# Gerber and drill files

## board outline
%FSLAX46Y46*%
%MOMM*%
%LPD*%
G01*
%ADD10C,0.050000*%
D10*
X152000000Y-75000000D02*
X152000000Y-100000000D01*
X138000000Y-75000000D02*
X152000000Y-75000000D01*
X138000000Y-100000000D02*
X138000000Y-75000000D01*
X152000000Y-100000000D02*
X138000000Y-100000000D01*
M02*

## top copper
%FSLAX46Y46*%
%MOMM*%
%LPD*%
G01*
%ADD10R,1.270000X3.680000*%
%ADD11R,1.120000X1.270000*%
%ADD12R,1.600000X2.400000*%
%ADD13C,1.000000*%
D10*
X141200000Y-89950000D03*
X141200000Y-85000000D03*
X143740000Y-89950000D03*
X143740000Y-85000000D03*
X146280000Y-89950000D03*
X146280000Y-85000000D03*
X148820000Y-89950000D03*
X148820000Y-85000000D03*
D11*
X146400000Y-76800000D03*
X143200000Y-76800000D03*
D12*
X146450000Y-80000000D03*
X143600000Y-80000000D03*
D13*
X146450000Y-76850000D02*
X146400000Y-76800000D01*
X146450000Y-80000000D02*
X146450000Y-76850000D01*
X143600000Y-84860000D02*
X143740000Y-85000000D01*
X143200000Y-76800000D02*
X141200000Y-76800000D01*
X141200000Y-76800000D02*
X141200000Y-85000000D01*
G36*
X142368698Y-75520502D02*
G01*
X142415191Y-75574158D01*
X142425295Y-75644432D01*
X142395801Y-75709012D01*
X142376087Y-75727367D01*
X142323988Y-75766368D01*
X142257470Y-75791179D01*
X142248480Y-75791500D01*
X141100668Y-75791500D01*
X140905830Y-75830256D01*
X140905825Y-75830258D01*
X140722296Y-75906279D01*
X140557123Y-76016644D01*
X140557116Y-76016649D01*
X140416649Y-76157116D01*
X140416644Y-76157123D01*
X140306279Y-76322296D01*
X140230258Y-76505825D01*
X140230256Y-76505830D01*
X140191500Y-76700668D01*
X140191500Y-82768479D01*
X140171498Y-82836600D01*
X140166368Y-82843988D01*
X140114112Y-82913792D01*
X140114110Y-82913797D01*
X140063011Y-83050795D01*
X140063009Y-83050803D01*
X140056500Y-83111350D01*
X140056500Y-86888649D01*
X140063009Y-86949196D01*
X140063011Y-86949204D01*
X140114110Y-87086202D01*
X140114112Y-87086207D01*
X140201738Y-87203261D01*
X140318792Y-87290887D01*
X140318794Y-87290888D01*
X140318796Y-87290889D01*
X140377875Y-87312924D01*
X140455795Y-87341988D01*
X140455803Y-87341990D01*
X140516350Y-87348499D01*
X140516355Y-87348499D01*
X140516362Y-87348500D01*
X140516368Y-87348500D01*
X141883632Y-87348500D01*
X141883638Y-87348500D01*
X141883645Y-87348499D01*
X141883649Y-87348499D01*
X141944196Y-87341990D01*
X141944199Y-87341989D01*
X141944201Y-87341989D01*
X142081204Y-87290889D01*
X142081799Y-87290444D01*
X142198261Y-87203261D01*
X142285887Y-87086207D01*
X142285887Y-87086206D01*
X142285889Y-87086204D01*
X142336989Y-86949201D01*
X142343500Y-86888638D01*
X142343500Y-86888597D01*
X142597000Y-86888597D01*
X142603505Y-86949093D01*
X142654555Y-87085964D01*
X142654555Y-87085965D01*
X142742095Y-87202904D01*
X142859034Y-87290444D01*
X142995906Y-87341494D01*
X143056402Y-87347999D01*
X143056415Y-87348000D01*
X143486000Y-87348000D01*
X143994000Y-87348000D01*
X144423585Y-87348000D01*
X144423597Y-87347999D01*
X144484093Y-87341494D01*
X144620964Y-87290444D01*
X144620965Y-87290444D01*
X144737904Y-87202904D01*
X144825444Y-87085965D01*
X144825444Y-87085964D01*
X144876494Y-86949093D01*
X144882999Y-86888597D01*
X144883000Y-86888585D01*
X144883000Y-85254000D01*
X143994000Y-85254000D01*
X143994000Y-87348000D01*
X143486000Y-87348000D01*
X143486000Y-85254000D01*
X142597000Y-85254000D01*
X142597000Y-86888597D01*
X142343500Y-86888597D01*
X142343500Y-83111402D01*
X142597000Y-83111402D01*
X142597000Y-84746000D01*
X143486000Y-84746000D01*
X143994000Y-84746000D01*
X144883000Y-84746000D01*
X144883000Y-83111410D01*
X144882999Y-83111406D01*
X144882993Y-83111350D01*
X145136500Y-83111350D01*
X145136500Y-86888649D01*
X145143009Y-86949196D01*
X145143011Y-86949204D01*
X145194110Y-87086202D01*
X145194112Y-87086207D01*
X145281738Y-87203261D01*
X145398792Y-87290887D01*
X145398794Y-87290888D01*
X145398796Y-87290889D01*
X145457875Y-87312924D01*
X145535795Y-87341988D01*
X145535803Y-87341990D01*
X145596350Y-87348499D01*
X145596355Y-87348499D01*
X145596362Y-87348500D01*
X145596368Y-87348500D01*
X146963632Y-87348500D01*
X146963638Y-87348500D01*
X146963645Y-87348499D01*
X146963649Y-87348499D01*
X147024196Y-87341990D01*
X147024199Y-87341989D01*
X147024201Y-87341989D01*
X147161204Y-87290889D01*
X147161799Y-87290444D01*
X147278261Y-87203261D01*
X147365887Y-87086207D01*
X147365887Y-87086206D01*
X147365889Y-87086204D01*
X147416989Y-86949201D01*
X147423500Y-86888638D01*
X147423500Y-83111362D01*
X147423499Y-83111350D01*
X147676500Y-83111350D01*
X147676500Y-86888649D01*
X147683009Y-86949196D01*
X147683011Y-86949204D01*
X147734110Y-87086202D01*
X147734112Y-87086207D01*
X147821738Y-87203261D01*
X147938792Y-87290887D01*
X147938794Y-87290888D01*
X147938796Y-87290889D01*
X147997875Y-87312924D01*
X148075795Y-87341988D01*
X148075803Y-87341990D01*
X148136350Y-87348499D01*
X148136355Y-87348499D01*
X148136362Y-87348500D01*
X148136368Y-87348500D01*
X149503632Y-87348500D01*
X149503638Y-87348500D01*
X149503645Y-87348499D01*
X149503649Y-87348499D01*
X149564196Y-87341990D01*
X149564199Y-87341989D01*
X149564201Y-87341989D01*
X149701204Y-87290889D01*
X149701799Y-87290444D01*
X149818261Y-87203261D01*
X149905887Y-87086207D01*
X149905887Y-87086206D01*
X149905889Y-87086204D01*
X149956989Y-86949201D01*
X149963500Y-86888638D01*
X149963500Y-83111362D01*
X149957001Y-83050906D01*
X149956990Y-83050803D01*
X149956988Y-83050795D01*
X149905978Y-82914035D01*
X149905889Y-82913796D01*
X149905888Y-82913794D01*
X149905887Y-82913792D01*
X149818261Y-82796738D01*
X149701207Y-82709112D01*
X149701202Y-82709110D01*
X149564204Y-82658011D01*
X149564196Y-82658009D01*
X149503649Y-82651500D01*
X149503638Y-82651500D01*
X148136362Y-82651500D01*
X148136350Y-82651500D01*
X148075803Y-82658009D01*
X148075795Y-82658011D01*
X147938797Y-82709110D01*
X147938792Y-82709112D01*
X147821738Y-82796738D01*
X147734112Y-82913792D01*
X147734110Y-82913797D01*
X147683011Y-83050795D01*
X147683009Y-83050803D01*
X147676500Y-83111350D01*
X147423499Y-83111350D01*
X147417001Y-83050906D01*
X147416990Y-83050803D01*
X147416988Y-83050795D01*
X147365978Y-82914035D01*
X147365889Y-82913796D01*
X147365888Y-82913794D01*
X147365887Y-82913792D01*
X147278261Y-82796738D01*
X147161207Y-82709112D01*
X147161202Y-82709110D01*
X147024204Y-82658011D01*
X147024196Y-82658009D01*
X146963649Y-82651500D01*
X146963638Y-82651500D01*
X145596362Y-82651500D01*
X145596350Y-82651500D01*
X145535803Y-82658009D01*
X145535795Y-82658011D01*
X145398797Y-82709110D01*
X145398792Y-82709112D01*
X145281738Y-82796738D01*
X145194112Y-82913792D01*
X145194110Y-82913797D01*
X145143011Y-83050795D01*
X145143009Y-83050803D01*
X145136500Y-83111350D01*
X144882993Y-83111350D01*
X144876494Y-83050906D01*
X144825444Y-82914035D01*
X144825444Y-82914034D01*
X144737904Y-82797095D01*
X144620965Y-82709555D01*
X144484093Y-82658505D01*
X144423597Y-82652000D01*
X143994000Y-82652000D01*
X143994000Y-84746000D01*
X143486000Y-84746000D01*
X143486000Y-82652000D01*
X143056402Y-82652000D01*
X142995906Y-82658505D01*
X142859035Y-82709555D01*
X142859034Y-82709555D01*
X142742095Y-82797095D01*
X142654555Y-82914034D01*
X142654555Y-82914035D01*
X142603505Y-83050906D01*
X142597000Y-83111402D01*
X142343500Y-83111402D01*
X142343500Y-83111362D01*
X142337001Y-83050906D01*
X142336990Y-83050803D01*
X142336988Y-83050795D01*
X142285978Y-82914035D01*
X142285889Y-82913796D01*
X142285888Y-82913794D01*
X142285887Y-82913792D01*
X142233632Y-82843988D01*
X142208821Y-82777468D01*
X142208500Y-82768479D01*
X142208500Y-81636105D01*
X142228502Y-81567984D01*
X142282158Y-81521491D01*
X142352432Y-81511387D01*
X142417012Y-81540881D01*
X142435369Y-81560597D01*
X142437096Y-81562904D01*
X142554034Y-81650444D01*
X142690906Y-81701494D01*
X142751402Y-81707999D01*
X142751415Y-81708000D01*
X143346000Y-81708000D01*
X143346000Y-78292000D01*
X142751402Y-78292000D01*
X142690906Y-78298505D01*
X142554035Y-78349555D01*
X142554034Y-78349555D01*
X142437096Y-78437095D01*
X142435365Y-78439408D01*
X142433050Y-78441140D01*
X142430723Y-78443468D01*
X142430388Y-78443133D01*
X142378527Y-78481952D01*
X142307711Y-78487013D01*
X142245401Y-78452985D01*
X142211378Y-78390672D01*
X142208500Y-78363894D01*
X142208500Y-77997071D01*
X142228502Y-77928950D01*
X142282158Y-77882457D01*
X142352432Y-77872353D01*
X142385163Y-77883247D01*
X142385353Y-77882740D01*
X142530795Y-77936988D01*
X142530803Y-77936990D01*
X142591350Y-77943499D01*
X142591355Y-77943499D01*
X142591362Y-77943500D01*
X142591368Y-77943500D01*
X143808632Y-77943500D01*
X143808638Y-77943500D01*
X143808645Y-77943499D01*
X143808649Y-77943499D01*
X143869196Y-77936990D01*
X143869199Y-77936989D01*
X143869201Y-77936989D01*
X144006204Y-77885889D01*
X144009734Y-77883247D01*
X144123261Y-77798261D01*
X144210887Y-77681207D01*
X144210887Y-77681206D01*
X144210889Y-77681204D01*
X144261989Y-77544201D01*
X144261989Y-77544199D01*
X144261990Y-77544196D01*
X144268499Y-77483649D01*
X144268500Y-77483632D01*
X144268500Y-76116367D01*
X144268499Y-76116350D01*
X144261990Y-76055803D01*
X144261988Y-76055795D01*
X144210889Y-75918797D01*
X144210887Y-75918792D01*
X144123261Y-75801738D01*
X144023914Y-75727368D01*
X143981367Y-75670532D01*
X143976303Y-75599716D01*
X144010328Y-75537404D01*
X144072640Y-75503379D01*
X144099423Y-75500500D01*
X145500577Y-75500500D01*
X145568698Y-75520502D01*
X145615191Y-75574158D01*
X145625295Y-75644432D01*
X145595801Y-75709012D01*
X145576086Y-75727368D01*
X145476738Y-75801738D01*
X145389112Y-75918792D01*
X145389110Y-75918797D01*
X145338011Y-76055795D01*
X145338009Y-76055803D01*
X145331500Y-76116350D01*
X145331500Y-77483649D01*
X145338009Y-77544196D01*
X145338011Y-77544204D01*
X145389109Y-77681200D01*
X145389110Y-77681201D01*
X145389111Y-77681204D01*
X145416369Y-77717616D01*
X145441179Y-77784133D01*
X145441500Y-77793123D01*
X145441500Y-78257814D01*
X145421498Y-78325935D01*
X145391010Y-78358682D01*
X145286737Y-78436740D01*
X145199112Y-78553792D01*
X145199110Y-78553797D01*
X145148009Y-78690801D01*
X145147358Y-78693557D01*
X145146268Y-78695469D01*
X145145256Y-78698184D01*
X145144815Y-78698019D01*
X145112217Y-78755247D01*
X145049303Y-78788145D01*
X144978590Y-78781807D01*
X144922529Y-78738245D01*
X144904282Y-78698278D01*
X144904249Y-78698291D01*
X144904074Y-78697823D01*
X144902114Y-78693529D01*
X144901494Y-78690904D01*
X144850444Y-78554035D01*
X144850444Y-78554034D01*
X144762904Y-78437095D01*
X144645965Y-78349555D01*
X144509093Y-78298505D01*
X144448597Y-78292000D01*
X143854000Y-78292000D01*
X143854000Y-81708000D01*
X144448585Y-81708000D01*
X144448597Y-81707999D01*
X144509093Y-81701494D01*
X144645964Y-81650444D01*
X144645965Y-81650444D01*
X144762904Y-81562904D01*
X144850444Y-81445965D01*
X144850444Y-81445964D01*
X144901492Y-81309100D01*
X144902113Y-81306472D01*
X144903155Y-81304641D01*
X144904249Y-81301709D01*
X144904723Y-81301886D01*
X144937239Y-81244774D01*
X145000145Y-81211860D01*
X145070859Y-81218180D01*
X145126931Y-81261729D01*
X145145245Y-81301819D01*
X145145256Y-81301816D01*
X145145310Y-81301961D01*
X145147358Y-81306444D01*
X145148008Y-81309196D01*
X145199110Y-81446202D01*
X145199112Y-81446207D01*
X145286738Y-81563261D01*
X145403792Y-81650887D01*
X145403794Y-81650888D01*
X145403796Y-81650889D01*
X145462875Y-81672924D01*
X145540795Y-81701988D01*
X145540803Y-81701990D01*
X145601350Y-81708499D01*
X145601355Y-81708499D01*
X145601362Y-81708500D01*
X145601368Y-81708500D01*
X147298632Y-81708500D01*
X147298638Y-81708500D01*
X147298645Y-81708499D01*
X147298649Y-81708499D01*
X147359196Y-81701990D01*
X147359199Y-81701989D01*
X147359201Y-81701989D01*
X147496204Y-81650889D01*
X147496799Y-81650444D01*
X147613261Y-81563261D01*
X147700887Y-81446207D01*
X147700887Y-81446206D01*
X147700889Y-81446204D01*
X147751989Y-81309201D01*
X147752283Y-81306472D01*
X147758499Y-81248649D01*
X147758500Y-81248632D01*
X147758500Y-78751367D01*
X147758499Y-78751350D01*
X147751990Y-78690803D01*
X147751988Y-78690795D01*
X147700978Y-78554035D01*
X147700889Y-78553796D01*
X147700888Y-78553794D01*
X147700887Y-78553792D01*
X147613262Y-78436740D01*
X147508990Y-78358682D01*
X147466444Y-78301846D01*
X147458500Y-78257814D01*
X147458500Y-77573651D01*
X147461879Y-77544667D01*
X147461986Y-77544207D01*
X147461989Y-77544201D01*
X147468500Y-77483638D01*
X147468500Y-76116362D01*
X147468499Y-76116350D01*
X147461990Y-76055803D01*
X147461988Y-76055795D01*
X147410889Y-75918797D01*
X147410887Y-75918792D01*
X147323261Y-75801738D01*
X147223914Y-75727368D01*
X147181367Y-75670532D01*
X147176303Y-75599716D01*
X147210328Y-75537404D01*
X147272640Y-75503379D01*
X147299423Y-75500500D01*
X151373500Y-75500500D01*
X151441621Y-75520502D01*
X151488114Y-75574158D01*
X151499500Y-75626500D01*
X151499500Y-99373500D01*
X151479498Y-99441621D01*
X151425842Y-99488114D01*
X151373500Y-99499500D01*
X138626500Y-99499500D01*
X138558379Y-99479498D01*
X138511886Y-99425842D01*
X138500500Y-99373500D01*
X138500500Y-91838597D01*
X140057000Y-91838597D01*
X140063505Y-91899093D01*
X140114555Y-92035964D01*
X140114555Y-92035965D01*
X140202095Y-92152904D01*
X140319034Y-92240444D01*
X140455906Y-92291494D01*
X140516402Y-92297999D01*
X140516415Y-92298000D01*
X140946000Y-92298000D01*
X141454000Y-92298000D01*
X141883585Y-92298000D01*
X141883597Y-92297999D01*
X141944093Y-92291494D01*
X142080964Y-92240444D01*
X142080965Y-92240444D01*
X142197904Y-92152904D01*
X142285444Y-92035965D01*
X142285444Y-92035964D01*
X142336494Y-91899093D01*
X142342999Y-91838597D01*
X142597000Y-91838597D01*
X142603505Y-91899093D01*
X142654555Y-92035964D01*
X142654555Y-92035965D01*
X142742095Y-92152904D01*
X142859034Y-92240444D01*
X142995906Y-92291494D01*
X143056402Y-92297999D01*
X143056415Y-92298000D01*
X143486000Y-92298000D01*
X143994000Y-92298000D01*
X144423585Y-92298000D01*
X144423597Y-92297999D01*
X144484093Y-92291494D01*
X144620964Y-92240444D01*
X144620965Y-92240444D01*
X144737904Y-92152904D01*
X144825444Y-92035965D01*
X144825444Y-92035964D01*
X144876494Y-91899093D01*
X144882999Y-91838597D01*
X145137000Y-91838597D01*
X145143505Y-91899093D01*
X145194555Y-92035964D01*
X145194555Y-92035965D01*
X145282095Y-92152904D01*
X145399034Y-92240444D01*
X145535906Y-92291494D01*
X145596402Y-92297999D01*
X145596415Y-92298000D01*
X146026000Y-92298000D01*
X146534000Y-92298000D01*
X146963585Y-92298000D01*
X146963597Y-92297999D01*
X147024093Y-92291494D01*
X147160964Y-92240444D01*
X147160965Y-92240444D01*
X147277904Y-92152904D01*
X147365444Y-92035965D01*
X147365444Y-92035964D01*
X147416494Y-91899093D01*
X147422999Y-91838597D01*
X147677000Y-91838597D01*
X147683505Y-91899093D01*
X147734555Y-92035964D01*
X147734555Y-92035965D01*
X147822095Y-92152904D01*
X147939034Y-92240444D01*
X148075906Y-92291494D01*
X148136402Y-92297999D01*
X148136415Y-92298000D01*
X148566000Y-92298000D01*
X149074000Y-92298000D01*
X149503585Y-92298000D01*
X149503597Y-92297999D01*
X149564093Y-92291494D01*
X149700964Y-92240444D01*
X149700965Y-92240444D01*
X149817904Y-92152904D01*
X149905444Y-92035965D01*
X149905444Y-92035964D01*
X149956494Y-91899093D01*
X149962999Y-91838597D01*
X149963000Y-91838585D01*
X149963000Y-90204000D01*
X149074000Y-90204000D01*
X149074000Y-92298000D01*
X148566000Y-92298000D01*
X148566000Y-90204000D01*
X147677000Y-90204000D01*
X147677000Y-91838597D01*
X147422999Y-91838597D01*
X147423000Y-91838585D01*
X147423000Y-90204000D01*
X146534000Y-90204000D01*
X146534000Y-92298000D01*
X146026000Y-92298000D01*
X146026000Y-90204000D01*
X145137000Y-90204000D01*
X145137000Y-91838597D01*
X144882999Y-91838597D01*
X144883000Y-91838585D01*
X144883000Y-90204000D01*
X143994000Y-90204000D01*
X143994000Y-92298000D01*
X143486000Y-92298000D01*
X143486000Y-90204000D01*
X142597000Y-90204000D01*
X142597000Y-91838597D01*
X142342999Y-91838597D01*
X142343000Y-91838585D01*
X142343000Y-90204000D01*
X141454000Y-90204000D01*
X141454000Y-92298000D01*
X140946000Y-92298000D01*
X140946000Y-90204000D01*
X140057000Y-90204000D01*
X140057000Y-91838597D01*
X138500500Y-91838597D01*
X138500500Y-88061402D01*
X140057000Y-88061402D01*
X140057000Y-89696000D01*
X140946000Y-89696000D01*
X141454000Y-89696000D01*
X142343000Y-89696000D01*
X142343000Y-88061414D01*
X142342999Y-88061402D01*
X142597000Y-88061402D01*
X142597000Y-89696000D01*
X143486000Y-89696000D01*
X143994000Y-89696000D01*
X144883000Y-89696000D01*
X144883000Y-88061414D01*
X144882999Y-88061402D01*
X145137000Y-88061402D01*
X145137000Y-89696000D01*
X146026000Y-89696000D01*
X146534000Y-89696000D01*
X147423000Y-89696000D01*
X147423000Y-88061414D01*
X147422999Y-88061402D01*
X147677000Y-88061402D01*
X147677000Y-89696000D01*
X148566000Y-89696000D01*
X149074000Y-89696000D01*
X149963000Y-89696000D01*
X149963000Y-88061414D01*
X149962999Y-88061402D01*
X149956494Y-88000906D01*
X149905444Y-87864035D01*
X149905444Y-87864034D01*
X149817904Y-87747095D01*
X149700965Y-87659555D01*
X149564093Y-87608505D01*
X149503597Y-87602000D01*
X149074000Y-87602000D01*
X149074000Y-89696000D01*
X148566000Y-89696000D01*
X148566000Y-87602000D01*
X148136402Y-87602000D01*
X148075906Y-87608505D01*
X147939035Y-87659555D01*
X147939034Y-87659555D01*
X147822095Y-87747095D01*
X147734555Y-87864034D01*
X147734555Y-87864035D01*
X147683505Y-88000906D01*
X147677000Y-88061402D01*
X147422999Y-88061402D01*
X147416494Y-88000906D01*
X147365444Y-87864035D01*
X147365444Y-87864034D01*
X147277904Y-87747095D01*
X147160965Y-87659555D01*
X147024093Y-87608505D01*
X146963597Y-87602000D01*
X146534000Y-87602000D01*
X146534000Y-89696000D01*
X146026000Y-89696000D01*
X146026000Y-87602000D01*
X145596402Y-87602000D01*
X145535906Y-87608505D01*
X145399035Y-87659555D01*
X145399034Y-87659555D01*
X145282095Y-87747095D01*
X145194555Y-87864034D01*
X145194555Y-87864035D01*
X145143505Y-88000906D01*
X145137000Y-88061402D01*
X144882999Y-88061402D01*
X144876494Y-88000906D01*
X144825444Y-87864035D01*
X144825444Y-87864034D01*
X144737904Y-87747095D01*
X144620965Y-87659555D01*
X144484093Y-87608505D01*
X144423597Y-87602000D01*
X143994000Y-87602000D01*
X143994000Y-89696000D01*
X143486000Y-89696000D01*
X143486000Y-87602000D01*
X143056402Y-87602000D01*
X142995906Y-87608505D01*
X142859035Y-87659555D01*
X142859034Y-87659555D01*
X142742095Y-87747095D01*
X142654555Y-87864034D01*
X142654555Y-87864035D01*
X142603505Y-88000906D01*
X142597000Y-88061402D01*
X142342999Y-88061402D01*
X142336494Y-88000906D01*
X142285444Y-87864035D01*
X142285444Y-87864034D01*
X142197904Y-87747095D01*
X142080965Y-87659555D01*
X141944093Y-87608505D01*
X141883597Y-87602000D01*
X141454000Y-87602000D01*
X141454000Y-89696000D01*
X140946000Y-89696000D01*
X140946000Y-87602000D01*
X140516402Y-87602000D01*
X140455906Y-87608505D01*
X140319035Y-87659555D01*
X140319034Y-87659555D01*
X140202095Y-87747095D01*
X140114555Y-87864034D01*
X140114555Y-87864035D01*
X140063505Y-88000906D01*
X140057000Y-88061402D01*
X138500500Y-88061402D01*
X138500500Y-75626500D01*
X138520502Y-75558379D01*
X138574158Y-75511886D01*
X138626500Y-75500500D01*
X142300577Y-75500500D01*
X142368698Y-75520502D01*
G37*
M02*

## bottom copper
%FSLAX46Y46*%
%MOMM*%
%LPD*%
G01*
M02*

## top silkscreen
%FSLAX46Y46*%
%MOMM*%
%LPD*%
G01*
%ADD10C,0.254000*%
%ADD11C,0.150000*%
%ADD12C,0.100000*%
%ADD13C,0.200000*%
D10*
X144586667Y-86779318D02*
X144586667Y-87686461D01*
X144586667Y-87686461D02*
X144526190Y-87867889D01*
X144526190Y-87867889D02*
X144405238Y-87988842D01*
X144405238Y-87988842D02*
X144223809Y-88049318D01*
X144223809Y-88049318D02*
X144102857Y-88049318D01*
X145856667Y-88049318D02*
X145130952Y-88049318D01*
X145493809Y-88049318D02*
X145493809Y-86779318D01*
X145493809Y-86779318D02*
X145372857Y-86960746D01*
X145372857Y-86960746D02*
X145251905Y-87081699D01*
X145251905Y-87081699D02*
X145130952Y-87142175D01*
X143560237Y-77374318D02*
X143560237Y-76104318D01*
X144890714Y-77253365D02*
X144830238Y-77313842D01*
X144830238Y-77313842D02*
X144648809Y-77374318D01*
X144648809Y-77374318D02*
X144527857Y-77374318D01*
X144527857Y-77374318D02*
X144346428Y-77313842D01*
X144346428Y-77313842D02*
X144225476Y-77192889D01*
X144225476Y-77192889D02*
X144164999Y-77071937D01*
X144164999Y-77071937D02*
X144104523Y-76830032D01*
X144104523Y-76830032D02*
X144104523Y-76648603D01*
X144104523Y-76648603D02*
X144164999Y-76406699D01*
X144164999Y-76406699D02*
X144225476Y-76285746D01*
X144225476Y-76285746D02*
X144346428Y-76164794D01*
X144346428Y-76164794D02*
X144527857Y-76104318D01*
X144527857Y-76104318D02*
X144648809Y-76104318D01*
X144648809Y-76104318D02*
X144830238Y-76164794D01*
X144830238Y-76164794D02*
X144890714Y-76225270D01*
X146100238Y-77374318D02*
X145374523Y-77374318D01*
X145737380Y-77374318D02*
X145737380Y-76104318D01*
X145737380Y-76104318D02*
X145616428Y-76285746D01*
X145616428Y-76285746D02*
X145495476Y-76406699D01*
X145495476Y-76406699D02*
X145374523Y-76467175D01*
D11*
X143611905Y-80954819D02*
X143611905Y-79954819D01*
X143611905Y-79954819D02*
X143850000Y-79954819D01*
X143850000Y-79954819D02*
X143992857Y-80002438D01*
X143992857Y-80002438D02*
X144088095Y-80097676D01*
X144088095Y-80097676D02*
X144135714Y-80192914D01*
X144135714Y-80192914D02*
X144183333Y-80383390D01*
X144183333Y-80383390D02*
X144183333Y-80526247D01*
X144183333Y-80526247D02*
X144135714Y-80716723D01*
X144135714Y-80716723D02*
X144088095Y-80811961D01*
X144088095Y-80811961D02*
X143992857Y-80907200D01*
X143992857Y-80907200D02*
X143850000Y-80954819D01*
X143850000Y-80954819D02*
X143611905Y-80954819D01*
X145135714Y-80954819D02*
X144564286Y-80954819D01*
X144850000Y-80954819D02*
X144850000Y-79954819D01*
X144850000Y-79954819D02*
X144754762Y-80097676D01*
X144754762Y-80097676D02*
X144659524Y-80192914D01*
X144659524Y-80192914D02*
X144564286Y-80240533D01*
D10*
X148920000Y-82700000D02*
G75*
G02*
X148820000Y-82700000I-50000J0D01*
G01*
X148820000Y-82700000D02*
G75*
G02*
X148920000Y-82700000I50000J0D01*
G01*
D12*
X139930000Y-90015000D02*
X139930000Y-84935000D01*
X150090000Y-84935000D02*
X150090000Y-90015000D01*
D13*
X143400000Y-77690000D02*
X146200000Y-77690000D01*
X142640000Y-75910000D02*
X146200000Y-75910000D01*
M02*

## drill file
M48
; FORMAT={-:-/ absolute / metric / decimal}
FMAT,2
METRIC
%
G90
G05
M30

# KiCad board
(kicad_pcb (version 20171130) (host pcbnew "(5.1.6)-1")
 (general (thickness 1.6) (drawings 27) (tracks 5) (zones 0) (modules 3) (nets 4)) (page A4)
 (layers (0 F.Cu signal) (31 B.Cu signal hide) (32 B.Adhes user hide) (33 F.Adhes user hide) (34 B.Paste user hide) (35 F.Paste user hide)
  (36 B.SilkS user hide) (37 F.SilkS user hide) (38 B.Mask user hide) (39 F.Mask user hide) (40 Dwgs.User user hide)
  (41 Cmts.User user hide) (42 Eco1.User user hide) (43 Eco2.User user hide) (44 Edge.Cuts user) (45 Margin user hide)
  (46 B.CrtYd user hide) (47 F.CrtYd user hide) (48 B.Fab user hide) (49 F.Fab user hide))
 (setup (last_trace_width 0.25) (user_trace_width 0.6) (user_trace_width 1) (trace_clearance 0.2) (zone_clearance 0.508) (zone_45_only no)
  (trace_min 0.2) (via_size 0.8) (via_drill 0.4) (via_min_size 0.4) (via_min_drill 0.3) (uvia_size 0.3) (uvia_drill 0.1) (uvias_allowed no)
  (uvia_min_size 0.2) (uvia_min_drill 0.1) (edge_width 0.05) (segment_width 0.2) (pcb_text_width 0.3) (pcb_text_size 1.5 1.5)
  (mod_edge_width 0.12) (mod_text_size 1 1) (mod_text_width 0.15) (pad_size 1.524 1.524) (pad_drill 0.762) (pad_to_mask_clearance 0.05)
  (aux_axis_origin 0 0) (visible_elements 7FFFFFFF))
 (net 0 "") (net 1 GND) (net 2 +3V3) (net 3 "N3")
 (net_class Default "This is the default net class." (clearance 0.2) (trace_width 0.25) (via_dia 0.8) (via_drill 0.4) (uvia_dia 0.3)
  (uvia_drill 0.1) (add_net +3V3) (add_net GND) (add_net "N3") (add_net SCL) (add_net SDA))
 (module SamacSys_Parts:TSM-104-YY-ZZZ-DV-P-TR (layer F.Cu) (at 145.01 87.475)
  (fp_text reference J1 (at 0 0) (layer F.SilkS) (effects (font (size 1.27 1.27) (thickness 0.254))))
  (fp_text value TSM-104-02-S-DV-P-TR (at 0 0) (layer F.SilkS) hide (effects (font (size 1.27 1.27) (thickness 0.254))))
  (fp_circle (center 3.86 -4.775) (end 3.81 -4.775) (layer F.SilkS) (width 0.254))
  (fp_line (start -5.08 2.54) (end -5.08 -2.54) (layer F.SilkS) (width 0.1))
  (fp_line (start 5.08 -2.54) (end 5.08 2.54) (layer F.SilkS) (width 0.1))
  (pad 8 smd rect (at -3.81 2.475) (size 1.27 3.68) (layers F.Cu F.Paste F.Mask) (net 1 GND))
  (pad 7 smd rect (at -3.81 -2.475) (size 1.27 3.68) (layers F.Cu F.Paste F.Mask) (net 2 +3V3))
  (pad 6 smd rect (at -1.27 2.475) (size 1.27 3.68) (layers F.Cu F.Paste F.Mask) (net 1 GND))
  (pad 5 smd rect (at -1.27 -2.475) (size 1.27 3.68) (layers F.Cu F.Paste F.Mask) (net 1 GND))
  (pad 4 smd rect (at 1.27 2.475) (size 1.27 3.68) (layers F.Cu F.Paste F.Mask) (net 1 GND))
  (pad 3 smd rect (at 1.27 -2.475) (size 1.27 3.68) (layers F.Cu F.Paste F.Mask))
  (pad 2 smd rect (at 3.81 2.475) (size 1.27 3.68) (layers F.Cu F.Paste F.Mask) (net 1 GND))
  (pad 1 smd rect (at 3.81 -2.475) (size 1.27 3.68) (layers F.Cu F.Paste F.Mask)))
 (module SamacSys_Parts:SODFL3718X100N (layer F.Cu) (at 144.8 76.8)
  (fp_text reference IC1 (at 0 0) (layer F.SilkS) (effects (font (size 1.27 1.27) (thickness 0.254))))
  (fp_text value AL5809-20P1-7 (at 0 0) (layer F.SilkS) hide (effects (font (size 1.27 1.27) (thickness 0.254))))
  (fp_line (start -1.4 0.89) (end 1.4 0.89) (layer F.SilkS) (width 0.2))
  (fp_line (start -2.16 -0.89) (end 1.4 -0.89) (layer F.SilkS) (width 0.2))
  (pad 2 smd rect (at 1.6 0) (size 1.12 1.27) (layers F.Cu F.Paste F.Mask) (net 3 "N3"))
  (pad 1 smd rect (at -1.6 0) (size 1.12 1.27) (layers F.Cu F.Paste F.Mask) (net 2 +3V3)))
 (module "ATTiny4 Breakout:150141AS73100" (layer F.Cu) (at 144.35 80)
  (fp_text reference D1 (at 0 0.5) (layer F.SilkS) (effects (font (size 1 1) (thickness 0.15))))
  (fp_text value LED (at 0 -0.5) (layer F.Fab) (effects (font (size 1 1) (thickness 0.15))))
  (pad 2 smd rect (at 2.1 0) (size 1.6 2.4) (layers F.Cu F.Paste F.Mask) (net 3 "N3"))
  (pad 1 smd rect (at -0.75 0) (size 1.6 2.4) (layers F.Cu F.Paste F.Mask) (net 1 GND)))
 (gr_line (start 152 75) (end 152 100) (layer Edge.Cuts) (width 0.05))
 (gr_line (start 138 75) (end 152 75) (layer Edge.Cuts) (width 0.05))
 (gr_line (start 138 100) (end 138 75) (layer Edge.Cuts) (width 0.05))
 (gr_line (start 152 100) (end 138 100) (layer Edge.Cuts) (width 0.05))
 (segment (start 146.45 76.85) (end 146.4 76.8) (width 1) (layer F.Cu) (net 3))
 (segment (start 146.45 80) (end 146.45 76.85) (width 1) (layer F.Cu) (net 3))
 (segment (start 143.6 84.86) (end 143.74 85) (width 1) (layer F.Cu) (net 1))
 (segment (start 143.2 76.8) (end 141.2 76.8) (width 1) (layer F.Cu) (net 2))
 (segment (start 141.2 76.8) (end 141.2 85) (width 1) (layer F.Cu) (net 2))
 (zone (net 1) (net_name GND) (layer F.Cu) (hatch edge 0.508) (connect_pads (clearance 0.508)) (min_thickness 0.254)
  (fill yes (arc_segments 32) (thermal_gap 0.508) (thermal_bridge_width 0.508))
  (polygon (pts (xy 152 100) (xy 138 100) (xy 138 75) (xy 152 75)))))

